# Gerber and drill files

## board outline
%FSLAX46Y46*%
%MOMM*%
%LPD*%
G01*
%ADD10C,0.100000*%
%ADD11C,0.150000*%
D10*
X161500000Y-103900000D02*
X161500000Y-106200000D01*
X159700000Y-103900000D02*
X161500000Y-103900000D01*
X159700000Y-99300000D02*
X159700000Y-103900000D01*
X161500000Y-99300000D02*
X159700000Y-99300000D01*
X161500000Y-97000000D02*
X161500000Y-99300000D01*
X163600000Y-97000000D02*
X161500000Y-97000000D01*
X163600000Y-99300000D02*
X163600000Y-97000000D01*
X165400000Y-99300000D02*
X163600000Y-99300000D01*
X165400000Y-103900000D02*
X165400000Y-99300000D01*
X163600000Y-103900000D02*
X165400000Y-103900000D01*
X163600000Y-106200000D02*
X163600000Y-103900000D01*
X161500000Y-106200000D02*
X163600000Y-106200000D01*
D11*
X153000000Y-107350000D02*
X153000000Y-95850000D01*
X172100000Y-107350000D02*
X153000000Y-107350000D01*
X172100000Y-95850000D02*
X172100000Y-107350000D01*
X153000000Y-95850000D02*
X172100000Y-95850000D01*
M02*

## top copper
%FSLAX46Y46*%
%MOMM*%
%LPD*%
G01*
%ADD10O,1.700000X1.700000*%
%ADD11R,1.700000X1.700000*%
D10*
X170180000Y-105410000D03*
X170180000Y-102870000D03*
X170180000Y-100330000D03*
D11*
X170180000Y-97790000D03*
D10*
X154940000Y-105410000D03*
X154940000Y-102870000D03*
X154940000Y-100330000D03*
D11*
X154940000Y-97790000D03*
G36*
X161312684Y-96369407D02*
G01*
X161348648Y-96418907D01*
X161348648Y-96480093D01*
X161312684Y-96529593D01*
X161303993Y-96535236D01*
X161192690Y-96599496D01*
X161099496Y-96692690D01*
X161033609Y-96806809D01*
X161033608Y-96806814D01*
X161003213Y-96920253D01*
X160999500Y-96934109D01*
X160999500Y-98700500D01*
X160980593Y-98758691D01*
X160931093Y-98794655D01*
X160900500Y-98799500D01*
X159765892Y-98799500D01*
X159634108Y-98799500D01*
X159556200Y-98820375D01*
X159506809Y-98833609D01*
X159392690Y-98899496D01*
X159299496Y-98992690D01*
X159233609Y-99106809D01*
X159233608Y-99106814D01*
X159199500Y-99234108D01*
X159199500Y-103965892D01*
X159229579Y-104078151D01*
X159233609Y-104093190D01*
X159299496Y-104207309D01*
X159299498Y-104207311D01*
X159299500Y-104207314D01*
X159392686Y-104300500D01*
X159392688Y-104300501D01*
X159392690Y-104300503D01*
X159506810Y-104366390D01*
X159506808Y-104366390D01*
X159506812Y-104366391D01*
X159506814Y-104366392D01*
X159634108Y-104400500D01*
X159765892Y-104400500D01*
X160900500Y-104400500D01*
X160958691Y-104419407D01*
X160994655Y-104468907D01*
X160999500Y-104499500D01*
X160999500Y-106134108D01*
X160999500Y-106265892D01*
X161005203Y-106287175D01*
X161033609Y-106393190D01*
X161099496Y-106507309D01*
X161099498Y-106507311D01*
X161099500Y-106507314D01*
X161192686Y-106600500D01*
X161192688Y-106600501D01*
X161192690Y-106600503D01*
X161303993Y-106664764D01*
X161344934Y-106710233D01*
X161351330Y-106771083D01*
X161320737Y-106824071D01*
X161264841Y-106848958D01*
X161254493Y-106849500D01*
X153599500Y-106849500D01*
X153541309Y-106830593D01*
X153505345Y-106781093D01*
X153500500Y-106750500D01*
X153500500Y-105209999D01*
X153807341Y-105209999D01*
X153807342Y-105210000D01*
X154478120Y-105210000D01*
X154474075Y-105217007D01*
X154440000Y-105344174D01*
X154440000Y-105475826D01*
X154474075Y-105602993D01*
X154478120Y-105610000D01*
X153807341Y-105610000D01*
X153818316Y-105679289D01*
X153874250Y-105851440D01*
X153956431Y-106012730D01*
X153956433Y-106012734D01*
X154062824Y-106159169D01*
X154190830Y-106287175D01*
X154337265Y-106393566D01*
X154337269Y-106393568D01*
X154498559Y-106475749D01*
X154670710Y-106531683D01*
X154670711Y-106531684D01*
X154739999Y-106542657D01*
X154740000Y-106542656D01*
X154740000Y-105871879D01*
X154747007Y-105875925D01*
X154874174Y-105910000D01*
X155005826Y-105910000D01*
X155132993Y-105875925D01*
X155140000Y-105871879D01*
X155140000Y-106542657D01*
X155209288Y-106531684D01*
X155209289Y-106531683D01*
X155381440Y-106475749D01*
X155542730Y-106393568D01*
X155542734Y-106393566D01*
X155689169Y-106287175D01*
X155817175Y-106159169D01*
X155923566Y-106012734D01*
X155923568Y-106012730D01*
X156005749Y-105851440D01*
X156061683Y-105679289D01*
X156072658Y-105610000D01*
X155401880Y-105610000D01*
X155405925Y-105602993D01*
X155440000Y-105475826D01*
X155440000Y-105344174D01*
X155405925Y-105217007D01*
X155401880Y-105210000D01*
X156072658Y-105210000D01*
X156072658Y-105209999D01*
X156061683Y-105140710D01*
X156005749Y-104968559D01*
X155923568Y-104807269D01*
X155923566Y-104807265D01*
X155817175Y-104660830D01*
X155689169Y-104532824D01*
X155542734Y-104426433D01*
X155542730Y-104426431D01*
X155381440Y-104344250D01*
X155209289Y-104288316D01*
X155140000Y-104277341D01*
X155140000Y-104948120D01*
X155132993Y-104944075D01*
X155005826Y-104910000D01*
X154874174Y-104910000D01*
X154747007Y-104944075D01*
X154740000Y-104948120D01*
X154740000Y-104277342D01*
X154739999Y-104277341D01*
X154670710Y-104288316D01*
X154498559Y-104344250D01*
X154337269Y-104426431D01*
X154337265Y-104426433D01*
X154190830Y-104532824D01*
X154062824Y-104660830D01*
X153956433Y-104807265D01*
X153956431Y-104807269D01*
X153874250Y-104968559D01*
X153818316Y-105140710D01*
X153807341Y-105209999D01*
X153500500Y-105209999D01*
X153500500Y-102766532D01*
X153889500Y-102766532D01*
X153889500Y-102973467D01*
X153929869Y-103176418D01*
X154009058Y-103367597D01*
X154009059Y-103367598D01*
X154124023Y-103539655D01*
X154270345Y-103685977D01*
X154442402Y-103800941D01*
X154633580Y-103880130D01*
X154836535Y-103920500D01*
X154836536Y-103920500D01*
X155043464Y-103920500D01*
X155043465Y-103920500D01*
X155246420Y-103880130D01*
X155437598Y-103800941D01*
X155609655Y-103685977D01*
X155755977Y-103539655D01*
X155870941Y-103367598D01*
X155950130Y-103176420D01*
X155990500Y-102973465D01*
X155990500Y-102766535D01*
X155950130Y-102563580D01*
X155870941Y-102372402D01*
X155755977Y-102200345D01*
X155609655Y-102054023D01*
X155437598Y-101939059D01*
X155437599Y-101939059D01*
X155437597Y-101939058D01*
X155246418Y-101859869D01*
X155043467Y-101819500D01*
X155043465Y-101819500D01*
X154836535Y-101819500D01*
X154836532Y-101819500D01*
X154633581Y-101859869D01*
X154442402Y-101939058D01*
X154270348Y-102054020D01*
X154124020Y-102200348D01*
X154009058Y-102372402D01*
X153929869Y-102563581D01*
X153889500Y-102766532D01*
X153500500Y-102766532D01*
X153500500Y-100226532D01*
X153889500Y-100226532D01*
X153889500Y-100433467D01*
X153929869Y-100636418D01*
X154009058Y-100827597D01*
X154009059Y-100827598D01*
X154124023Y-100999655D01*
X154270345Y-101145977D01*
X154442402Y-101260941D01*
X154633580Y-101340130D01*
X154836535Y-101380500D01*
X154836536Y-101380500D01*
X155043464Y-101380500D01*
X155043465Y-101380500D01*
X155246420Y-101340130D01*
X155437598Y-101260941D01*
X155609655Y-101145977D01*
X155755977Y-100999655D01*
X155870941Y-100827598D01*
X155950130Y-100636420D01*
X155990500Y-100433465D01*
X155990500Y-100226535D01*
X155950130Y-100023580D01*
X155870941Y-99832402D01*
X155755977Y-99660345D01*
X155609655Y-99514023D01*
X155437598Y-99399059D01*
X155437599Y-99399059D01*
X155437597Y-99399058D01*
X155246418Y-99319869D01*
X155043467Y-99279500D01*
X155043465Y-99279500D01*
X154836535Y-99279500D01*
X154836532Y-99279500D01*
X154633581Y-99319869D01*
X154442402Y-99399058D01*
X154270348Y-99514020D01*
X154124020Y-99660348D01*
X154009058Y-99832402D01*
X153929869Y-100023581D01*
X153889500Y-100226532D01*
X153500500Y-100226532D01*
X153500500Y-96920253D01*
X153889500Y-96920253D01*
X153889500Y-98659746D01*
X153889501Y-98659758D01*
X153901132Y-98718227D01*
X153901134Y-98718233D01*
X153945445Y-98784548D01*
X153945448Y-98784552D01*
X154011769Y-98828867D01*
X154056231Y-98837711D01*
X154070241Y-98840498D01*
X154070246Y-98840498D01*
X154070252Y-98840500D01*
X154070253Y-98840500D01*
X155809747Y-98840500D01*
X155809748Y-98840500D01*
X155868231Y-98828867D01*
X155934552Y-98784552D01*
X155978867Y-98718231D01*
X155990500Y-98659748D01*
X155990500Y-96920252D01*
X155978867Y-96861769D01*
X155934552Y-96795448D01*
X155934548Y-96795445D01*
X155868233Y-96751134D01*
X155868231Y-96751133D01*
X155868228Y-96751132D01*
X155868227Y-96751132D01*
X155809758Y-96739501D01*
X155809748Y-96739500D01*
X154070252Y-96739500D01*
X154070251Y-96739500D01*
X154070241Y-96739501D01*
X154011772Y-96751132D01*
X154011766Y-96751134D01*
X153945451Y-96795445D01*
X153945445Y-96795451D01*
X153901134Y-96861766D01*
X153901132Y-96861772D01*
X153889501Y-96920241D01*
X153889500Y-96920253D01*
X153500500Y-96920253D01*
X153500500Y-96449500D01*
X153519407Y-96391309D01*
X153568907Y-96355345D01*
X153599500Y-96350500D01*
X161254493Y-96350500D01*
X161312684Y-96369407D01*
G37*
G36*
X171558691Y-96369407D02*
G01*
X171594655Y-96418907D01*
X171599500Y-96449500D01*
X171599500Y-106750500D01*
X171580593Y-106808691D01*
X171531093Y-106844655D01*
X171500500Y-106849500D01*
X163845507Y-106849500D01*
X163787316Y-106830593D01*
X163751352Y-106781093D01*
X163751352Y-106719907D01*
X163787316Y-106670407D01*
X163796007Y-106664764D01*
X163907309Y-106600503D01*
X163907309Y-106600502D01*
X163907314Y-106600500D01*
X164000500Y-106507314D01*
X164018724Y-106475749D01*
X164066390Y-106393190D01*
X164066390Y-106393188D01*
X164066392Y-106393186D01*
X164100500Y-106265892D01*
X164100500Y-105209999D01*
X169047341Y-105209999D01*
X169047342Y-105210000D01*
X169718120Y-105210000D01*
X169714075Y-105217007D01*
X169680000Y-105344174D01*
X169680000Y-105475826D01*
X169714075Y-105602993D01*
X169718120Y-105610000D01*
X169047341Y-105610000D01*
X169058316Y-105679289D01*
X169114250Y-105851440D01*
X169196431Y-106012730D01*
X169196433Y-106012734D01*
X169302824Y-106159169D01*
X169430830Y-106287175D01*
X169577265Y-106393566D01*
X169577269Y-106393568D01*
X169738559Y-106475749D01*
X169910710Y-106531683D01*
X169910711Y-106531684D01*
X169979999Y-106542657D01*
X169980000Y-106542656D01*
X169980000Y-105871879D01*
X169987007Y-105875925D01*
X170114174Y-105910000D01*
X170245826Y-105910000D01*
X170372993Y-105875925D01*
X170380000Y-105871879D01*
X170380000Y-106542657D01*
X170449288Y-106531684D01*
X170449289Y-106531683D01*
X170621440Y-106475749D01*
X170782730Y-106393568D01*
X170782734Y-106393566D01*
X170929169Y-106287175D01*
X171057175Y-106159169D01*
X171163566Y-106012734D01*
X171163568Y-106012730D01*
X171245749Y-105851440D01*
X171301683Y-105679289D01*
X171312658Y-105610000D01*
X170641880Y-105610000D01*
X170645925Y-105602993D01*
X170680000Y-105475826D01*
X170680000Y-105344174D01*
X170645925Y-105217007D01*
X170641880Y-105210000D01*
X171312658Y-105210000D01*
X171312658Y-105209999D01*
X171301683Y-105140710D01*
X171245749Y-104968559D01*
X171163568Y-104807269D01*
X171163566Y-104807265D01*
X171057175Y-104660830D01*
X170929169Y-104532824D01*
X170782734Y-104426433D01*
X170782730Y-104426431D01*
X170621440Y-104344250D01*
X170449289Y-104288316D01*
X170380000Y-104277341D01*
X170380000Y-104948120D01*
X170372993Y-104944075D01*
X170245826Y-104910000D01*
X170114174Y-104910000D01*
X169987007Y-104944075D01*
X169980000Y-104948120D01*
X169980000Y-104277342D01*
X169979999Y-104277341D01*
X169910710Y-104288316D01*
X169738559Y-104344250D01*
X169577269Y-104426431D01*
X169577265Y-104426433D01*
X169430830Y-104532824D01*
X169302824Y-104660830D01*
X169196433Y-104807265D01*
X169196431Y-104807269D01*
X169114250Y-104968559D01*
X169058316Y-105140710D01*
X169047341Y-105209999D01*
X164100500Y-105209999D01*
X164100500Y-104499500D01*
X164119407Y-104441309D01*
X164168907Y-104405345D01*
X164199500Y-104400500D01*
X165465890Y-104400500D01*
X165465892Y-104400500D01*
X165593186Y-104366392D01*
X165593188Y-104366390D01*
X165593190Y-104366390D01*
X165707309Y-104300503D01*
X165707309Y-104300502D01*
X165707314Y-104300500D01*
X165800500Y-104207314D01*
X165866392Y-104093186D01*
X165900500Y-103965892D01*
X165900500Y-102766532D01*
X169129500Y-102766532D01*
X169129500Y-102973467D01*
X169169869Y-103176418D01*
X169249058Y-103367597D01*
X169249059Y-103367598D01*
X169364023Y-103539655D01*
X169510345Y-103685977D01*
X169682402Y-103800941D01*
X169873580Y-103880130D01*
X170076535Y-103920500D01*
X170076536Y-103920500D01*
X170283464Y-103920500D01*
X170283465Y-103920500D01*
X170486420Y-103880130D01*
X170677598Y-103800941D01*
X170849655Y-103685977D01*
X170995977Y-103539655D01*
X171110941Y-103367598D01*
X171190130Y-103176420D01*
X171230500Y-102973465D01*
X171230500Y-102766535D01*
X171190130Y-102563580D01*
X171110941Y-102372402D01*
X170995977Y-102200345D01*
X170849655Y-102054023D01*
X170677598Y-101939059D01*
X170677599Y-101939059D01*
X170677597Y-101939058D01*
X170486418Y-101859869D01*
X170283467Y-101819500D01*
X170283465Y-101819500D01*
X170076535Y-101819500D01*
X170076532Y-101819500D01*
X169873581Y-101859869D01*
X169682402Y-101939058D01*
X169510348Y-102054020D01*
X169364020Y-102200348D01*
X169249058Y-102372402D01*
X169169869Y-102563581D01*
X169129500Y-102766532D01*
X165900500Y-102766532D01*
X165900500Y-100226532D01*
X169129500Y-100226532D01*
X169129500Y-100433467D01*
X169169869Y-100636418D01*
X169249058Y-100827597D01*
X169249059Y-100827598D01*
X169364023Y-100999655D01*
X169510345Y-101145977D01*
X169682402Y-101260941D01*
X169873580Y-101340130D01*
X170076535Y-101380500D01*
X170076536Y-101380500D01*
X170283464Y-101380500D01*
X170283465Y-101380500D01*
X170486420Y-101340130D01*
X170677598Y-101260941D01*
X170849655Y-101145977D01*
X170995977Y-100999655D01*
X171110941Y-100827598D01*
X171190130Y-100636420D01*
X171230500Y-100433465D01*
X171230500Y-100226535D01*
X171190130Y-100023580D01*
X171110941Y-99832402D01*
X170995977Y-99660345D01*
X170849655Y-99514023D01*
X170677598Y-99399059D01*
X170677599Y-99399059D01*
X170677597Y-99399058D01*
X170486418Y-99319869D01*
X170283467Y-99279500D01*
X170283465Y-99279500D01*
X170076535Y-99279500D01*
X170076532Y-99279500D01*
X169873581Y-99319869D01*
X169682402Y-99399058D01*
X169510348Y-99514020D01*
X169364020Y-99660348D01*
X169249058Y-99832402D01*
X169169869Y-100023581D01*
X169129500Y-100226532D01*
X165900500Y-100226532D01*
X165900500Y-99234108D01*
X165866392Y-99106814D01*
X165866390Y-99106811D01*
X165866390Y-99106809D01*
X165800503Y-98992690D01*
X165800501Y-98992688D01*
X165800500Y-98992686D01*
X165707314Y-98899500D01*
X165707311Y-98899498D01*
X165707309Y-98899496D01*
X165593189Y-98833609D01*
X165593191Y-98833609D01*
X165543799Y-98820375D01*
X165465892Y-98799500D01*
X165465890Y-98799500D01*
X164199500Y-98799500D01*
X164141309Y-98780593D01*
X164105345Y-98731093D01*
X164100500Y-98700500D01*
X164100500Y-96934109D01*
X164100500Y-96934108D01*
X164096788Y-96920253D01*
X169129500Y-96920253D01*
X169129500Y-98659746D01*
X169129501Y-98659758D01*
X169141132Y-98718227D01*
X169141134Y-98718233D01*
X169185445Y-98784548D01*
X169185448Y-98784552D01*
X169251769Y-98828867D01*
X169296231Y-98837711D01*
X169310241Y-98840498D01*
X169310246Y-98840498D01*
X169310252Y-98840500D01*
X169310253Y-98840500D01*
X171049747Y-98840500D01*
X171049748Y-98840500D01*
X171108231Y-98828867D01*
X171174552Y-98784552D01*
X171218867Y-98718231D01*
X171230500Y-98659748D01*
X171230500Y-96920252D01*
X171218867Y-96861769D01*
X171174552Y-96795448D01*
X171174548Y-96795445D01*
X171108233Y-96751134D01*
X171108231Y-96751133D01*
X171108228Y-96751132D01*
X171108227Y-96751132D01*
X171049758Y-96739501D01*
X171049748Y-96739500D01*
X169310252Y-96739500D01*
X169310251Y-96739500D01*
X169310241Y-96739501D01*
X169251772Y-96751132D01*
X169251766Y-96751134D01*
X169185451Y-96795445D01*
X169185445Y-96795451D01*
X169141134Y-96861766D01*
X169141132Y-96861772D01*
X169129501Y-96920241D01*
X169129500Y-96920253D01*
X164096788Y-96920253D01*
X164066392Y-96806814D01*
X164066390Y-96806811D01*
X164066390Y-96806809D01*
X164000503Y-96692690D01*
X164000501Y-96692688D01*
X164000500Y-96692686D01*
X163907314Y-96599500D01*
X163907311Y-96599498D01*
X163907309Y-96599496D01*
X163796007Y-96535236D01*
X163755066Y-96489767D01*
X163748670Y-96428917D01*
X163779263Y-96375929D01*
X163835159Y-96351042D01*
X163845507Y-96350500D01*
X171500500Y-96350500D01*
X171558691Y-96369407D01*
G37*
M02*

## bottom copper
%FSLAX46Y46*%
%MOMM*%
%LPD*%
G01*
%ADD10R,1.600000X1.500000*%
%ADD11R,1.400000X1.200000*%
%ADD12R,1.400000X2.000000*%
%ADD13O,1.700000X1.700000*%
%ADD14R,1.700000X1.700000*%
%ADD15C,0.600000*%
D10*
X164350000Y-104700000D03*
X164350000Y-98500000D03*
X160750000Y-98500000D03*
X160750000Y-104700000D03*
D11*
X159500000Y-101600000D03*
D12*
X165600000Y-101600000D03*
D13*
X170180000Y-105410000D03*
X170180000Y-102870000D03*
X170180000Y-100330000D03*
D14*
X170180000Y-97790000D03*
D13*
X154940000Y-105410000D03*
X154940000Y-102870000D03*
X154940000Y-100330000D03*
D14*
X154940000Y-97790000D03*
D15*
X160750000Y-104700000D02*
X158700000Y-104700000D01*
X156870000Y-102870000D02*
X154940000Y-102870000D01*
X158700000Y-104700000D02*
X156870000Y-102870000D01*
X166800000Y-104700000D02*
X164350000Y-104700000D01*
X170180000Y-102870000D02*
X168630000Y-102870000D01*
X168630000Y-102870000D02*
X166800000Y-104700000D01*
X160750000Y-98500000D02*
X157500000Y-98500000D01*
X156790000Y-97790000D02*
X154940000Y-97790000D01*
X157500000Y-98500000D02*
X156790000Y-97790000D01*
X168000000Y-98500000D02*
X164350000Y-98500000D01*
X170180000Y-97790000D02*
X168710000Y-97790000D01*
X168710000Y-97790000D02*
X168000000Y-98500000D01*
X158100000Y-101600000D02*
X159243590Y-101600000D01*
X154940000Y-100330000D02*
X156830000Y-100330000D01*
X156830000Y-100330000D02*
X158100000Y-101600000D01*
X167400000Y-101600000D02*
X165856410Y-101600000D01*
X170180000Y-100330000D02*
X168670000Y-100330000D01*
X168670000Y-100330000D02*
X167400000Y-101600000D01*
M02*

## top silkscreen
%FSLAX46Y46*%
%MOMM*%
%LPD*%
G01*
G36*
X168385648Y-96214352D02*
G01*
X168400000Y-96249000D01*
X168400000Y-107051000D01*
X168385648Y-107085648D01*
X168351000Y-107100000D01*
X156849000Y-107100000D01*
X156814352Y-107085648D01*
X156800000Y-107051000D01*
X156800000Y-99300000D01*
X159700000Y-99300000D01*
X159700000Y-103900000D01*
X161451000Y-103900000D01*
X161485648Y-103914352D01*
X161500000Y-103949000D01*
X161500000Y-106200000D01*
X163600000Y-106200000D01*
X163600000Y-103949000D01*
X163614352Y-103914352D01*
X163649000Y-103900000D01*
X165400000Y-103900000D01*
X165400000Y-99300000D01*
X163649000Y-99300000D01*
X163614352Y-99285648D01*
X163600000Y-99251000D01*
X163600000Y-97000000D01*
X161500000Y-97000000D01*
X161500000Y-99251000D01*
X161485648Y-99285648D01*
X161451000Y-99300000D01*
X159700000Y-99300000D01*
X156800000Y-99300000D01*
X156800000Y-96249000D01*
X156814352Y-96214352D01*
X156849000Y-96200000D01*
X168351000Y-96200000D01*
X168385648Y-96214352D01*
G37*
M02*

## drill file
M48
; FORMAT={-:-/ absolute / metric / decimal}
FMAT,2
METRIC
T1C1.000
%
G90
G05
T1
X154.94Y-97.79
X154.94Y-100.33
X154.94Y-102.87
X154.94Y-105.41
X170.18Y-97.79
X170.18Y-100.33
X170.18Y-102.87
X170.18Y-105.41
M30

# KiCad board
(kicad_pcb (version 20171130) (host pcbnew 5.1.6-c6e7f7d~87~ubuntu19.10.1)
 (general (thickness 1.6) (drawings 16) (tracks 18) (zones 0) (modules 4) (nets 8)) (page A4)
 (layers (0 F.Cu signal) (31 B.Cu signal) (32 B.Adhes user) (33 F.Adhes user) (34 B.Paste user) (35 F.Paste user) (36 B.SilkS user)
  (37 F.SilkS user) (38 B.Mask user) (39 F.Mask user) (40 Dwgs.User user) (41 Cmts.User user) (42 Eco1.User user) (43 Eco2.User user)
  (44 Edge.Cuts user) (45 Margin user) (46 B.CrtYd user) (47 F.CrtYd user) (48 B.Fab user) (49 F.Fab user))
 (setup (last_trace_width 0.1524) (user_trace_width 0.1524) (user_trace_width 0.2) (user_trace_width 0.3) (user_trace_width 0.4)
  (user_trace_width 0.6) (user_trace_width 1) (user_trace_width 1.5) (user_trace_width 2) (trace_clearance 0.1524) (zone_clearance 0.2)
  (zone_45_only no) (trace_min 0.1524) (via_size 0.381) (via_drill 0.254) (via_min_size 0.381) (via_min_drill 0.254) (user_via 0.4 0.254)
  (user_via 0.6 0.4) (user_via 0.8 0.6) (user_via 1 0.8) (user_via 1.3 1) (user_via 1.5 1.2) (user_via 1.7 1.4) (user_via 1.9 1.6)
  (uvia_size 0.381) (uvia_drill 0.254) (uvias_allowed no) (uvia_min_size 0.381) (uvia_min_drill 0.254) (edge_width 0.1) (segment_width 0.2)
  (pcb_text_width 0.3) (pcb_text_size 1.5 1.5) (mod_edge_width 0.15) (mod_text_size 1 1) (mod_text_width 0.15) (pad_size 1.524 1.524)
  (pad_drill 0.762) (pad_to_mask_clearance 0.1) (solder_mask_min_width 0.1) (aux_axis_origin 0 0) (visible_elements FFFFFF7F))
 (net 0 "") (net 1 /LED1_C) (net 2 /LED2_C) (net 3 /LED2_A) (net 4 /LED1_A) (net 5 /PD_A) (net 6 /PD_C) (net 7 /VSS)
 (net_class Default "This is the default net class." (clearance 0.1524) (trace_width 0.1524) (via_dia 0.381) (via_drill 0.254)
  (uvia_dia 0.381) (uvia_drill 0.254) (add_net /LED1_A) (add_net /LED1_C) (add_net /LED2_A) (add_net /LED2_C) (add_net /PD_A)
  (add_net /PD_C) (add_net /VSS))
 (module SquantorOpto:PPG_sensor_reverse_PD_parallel (layer F.Cu) (at 162.55 101.6)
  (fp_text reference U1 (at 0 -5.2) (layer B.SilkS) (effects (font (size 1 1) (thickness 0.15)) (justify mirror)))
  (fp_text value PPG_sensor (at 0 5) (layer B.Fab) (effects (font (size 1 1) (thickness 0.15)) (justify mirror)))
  (pad 6 smd rect (at 1.8 3.1) (size 1.6 1.5) (layers B.Cu B.Paste B.Mask) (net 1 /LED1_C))
  (pad 4 smd rect (at 1.8 -3.1) (size 1.6 1.5) (layers B.Cu B.Paste B.Mask) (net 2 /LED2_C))
  (pad 3 smd rect (at -1.8 -3.1) (size 1.6 1.5) (layers B.Cu B.Paste B.Mask) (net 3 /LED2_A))
  (pad 1 smd rect (at -1.8 3.1) (size 1.6 1.5) (layers B.Cu B.Paste B.Mask) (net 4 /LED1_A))
  (pad 2 smd rect (at -3.05 0) (size 1.4 1.2) (layers B.Cu B.Paste B.Mask) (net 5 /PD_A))
  (pad 5 smd rect (at 3.05 0) (size 1.4 2) (layers B.Cu B.Paste B.Mask) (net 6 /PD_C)))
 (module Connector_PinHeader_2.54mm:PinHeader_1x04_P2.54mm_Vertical (layer B.Cu) (at 170.18 97.79 180)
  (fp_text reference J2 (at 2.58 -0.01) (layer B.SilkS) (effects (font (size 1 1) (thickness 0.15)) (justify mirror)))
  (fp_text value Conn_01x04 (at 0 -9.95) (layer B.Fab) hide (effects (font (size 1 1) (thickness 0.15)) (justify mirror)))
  (pad 4 thru_hole oval (at 0 -7.62 180) (size 1.7 1.7) (drill 1) (layers *.Cu *.Mask) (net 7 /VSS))
  (pad 3 thru_hole oval (at 0 -5.08 180) (size 1.7 1.7) (drill 1) (layers *.Cu *.Mask) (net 1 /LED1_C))
  (pad 2 thru_hole oval (at 0 -2.54 180) (size 1.7 1.7) (drill 1) (layers *.Cu *.Mask) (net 6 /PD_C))
  (pad 1 thru_hole rect (at 0 0 180) (size 1.7 1.7) (drill 1) (layers *.Cu *.Mask) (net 2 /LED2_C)))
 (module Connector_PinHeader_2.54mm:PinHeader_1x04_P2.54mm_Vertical (layer B.Cu) (at 154.94 97.79 180)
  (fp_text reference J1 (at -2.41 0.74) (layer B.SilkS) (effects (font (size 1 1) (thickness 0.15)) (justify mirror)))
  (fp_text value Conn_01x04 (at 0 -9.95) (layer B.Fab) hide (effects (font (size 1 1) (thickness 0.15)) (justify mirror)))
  (pad 4 thru_hole oval (at 0 -7.62 180) (size 1.7 1.7) (drill 1) (layers *.Cu *.Mask) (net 7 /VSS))
  (pad 3 thru_hole oval (at 0 -5.08 180) (size 1.7 1.7) (drill 1) (layers *.Cu *.Mask) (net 4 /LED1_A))
  (pad 2 thru_hole oval (at 0 -2.54 180) (size 1.7 1.7) (drill 1) (layers *.Cu *.Mask) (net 5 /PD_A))
  (pad 1 thru_hole rect (at 0 0 180) (size 1.7 1.7) (drill 1) (layers *.Cu *.Mask) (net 3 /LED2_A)))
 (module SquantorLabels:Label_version (layer B.Cu) (at 157.25 102.6 90)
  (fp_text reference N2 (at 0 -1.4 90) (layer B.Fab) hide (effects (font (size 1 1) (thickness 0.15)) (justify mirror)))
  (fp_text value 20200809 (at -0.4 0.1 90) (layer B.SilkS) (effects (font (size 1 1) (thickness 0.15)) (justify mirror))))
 (gr_line (start 161.5 103.9) (end 161.5 106.2) (layer Edge.Cuts) (width 0.1))
 (gr_line (start 159.7 103.9) (end 161.5 103.9) (layer Edge.Cuts) (width 0.1))
 (gr_line (start 159.7 99.3) (end 159.7 103.9) (layer Edge.Cuts) (width 0.1))
 (gr_line (start 161.5 99.3) (end 159.7 99.3) (layer Edge.Cuts) (width 0.1))
 (gr_line (start 161.5 97) (end 161.5 99.3) (layer Edge.Cuts) (width 0.1))
 (gr_line (start 163.6 97) (end 161.5 97) (layer Edge.Cuts) (width 0.1))
 (gr_line (start 163.6 99.3) (end 163.6 97) (layer Edge.Cuts) (width 0.1))
 (gr_line (start 165.4 99.3) (end 163.6 99.3) (layer Edge.Cuts) (width 0.1))
 (gr_line (start 165.4 103.9) (end 165.4 99.3) (layer Edge.Cuts) (width 0.1))
 (gr_line (start 163.6 103.9) (end 165.4 103.9) (layer Edge.Cuts) (width 0.1))
 (gr_line (start 163.6 106.2) (end 163.6 103.9) (layer Edge.Cuts) (width 0.1))
 (gr_line (start 161.5 106.2) (end 163.6 106.2) (layer Edge.Cuts) (width 0.1))
 (gr_line (start 153 107.35) (end 153 95.85) (layer Edge.Cuts) (width 0.15))
 (gr_line (start 172.1 107.35) (end 153 107.35) (layer Edge.Cuts) (width 0.15))
 (gr_line (start 172.1 95.85) (end 172.1 107.35) (layer Edge.Cuts) (width 0.15))
 (gr_line (start 153 95.85) (end 172.1 95.85) (layer Edge.Cuts) (width 0.15))
 (segment (start 160.75 104.7) (end 158.7 104.7) (width 0.6) (layer B.Cu) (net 4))
 (segment (start 156.87 102.87) (end 154.94 102.87) (width 0.6) (layer B.Cu) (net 4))
 (segment (start 158.7 104.7) (end 156.87 102.87) (width 0.6) (layer B.Cu) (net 4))
 (segment (start 166.8 104.7) (end 164.35 104.7) (width 0.6) (layer B.Cu) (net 1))
 (segment (start 170.18 102.87) (end 168.63 102.87) (width 0.6) (layer B.Cu) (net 1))
 (segment (start 168.63 102.87) (end 166.8 104.7) (width 0.6) (layer B.Cu) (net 1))
 (segment (start 160.75 98.5) (end 157.5 98.5) (width 0.6) (layer B.Cu) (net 3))
 (segment (start 156.79 97.79) (end 154.94 97.79) (width 0.6) (layer B.Cu) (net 3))
 (segment (start 157.5 98.5) (end 156.79 97.79) (width 0.6) (layer B.Cu) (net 3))
 (segment (start 168 98.5) (end 164.35 98.5) (width 0.6) (layer B.Cu) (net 2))
 (segment (start 170.18 97.79) (end 168.71 97.79) (width 0.6) (layer B.Cu) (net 2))
 (segment (start 168.71 97.79) (end 168 98.5) (width 0.6) (layer B.Cu) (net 2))
 (segment (start 158.1 101.6) (end 159.24359 101.6) (width 0.6) (layer B.Cu) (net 5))
 (segment (start 154.94 100.33) (end 156.83 100.33) (width 0.6) (layer B.Cu) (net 5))
 (segment (start 156.83 100.33) (end 158.1 101.6) (width 0.6) (layer B.Cu) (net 5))
 (segment (start 167.4 101.6) (end 165.85641 101.6) (width 0.6) (layer B.Cu) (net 6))
 (segment (start 170.18 100.33) (end 168.67 100.33) (width 0.6) (layer B.Cu) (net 6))
 (segment (start 168.67 100.33) (end 167.4 101.6) (width 0.6) (layer B.Cu) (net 6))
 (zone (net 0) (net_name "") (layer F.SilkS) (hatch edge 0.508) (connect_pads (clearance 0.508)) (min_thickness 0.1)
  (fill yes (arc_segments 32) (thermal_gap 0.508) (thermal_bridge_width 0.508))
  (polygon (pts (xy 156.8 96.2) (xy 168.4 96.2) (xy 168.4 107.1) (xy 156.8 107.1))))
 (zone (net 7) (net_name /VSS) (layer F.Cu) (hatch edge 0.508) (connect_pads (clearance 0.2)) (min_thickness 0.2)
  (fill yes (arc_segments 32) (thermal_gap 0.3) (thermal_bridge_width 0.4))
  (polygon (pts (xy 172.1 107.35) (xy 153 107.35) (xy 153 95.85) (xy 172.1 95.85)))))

